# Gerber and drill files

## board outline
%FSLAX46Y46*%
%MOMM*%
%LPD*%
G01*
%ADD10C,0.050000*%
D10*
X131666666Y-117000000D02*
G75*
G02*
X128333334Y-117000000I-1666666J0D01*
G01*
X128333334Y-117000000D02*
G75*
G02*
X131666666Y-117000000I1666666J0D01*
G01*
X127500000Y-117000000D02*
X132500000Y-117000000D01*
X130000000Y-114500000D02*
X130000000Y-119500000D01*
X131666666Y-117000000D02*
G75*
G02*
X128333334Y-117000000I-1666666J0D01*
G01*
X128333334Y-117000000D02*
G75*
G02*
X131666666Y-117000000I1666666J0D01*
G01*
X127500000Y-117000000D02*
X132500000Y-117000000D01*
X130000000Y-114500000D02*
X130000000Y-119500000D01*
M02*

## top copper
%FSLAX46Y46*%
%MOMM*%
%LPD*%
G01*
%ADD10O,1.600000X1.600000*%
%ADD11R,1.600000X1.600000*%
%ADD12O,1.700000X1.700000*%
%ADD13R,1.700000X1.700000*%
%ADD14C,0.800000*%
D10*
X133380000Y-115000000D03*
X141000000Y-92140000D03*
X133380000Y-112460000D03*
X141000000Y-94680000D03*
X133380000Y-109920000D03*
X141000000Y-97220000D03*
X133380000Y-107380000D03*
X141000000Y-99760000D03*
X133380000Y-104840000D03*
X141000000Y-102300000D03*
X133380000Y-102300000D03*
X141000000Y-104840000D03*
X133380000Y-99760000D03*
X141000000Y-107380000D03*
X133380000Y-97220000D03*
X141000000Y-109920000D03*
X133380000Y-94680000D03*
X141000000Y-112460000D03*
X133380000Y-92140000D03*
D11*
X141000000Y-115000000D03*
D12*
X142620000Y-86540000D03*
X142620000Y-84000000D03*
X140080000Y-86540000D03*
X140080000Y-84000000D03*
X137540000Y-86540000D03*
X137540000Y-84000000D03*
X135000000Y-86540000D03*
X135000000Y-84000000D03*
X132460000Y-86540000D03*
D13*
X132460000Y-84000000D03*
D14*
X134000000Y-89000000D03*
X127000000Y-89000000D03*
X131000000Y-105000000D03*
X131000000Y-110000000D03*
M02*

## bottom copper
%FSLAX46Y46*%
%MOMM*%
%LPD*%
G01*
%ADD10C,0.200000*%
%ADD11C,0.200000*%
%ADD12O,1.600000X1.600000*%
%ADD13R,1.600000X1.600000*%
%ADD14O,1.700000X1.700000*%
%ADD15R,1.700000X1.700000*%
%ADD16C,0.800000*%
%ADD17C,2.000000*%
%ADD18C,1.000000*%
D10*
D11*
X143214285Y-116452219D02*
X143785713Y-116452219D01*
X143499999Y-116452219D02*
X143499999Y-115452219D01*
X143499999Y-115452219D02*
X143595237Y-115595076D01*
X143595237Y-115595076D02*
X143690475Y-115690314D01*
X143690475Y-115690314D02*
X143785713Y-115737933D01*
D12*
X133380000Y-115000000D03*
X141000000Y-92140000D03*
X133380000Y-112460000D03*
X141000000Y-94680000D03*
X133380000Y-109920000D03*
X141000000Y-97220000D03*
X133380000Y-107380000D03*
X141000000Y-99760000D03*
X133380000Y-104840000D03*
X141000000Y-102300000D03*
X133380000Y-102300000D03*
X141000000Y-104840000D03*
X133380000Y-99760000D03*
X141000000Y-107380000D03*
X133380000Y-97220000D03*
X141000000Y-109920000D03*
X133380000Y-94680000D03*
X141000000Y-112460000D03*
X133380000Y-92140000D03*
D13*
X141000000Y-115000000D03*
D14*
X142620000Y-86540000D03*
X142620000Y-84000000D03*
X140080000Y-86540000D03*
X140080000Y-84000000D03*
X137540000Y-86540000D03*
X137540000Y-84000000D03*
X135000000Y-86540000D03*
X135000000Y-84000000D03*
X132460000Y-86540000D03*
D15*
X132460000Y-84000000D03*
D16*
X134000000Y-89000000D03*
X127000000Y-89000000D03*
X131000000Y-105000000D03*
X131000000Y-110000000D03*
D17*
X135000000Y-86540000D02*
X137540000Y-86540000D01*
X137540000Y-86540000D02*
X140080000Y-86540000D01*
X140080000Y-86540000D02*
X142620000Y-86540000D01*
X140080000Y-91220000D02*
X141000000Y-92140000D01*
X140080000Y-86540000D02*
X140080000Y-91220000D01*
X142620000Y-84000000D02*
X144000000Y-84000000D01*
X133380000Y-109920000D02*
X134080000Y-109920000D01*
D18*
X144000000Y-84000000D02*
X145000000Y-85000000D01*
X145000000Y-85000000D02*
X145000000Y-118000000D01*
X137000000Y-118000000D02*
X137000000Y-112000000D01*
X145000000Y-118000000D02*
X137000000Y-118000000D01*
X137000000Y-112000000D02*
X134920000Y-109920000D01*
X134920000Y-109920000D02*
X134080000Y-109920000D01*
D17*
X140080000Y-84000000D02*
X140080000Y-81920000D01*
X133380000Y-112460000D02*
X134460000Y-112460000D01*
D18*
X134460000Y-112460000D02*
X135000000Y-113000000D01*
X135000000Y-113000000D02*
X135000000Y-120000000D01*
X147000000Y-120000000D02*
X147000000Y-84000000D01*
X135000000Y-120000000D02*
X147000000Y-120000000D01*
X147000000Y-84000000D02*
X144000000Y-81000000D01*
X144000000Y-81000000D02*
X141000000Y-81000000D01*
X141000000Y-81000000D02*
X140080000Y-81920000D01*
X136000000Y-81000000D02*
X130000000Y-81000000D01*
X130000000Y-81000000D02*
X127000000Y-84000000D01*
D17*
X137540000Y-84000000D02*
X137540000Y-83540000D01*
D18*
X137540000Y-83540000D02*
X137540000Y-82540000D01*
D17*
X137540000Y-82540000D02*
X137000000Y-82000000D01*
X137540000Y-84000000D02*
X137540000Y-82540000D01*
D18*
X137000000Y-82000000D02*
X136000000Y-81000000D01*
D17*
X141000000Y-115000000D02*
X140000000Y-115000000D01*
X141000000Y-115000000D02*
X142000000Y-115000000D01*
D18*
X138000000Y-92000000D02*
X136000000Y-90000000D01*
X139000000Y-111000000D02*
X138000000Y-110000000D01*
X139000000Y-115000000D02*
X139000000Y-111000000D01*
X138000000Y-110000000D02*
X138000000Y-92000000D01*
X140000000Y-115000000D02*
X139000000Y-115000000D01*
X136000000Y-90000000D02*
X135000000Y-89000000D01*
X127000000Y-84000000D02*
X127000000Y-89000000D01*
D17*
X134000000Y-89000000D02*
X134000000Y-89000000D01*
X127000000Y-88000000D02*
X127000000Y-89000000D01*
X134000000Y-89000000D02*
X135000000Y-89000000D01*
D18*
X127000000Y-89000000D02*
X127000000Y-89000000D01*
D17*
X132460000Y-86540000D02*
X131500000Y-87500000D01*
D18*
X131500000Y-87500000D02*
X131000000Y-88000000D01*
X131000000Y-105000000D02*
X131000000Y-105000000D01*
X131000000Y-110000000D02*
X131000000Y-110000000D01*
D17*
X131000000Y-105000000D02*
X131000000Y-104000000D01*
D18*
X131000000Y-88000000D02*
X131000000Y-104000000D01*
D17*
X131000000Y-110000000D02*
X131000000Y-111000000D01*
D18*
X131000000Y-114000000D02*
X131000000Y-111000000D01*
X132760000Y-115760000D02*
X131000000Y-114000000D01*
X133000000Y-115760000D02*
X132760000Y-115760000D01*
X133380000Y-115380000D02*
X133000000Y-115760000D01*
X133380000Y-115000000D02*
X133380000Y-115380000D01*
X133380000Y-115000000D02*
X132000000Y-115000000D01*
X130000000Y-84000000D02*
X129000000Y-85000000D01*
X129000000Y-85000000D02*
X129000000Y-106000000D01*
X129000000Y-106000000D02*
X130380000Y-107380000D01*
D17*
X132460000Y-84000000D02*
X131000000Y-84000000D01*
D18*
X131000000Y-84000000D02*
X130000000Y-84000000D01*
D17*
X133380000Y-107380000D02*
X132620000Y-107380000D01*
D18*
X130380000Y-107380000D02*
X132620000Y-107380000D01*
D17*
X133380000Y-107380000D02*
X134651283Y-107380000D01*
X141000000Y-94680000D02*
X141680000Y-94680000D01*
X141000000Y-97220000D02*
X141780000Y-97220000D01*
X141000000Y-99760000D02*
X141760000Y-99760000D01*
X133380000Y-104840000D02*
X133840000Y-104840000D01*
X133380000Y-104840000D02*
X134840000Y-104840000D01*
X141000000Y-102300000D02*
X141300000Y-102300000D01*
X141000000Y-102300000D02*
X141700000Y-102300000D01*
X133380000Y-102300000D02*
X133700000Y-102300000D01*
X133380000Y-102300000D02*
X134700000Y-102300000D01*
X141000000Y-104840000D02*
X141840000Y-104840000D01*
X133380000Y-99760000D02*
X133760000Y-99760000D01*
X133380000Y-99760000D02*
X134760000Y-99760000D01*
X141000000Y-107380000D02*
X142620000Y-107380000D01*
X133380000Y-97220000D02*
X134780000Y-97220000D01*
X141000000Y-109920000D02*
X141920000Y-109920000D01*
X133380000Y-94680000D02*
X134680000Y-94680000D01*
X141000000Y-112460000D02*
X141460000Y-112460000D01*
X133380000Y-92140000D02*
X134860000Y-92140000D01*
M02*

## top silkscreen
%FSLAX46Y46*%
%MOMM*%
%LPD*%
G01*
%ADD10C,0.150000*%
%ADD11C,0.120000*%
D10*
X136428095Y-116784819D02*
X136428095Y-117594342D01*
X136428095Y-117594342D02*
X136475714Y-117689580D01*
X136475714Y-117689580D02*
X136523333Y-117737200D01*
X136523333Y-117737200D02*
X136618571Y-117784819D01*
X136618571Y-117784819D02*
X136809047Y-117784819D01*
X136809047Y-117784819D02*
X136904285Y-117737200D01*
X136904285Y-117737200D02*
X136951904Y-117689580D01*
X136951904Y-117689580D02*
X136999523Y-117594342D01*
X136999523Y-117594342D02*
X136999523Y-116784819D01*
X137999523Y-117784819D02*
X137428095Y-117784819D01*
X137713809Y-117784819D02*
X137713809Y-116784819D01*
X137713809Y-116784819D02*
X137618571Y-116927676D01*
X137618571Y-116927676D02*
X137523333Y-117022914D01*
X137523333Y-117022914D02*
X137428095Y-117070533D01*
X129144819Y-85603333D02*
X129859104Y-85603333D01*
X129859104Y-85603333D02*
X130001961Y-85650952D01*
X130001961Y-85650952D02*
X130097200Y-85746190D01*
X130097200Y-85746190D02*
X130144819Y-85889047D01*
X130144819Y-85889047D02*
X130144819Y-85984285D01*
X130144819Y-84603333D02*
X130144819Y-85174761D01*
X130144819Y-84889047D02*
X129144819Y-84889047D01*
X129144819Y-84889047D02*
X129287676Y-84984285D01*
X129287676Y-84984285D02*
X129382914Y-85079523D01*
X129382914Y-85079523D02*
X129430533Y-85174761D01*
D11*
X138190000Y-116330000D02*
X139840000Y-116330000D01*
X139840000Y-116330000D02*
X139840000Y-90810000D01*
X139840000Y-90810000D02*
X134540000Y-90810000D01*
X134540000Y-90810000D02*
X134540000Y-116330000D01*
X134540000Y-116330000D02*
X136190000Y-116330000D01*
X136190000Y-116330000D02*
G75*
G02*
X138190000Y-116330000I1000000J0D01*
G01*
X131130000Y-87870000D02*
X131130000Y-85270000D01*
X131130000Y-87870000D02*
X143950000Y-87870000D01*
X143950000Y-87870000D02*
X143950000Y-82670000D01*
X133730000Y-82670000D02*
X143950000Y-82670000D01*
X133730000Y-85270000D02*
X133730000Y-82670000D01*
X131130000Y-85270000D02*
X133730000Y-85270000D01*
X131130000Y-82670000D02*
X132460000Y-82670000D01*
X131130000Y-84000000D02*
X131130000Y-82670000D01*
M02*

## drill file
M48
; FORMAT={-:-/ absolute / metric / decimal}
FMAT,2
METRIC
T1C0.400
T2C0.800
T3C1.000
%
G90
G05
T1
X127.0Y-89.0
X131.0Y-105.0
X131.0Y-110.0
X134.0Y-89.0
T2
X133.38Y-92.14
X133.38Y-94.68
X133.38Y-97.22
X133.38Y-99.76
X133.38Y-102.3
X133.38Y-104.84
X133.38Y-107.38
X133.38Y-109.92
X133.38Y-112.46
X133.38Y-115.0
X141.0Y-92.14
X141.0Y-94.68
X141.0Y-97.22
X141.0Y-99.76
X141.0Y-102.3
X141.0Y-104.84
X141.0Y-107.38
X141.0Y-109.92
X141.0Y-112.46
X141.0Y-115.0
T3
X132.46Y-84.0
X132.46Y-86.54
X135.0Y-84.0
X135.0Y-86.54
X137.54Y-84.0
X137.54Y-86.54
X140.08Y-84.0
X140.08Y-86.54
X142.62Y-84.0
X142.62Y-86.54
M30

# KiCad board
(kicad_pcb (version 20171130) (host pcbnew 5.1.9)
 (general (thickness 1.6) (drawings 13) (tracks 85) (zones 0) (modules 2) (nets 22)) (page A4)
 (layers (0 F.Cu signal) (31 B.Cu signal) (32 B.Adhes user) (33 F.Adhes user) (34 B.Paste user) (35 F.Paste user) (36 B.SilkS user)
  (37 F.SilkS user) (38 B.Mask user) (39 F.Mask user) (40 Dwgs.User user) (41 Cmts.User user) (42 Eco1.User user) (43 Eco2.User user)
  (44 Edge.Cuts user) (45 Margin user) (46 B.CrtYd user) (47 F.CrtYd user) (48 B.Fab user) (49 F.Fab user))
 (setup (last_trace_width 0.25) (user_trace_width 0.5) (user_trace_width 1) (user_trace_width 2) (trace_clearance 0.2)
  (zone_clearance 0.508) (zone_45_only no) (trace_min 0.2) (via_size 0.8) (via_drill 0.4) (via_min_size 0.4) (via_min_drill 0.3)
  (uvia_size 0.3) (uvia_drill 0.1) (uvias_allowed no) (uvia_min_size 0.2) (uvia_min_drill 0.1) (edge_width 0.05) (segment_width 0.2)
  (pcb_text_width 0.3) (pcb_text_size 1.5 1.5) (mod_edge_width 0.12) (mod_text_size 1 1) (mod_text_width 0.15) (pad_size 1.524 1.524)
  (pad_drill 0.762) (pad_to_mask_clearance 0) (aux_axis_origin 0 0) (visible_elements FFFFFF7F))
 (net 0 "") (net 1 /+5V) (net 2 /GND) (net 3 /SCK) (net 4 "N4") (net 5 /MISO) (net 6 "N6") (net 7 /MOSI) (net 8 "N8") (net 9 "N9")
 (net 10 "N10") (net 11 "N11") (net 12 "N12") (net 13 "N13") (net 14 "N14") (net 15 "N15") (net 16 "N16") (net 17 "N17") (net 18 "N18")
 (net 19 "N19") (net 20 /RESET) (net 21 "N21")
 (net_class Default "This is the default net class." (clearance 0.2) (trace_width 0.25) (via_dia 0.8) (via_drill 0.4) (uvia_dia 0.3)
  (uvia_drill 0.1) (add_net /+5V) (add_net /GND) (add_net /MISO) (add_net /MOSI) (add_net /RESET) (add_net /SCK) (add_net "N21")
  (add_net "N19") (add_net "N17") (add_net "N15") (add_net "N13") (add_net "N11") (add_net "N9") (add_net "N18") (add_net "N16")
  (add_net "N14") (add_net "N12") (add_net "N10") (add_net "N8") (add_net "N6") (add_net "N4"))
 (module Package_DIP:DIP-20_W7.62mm (layer F.Cu) (at 141 115 180)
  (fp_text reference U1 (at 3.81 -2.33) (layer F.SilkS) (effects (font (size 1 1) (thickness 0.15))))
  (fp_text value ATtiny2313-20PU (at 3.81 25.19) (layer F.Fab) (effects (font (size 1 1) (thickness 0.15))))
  (fp_line (start 2.81 -1.33) (end 1.16 -1.33) (layer F.SilkS) (width 0.12))
  (fp_line (start 1.16 -1.33) (end 1.16 24.19) (layer F.SilkS) (width 0.12))
  (fp_line (start 1.16 24.19) (end 6.46 24.19) (layer F.SilkS) (width 0.12))
  (fp_line (start 6.46 24.19) (end 6.46 -1.33) (layer F.SilkS) (width 0.12))
  (fp_line (start 6.46 -1.33) (end 4.81 -1.33) (layer F.SilkS) (width 0.12))
  (fp_arc (start 3.81 -1.33) (end 2.81 -1.33) (angle -180) (layer F.SilkS) (width 0.12))
  (pad 20 thru_hole oval (at 7.62 0 180) (size 1.6 1.6) (drill 0.8) (layers *.Cu *.Mask) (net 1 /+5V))
  (pad 10 thru_hole oval (at 0 22.86 180) (size 1.6 1.6) (drill 0.8) (layers *.Cu *.Mask) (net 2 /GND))
  (pad 19 thru_hole oval (at 7.62 2.54 180) (size 1.6 1.6) (drill 0.8) (layers *.Cu *.Mask) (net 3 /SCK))
  (pad 9 thru_hole oval (at 0 20.32 180) (size 1.6 1.6) (drill 0.8) (layers *.Cu *.Mask) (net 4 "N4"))
  (pad 18 thru_hole oval (at 7.62 5.08 180) (size 1.6 1.6) (drill 0.8) (layers *.Cu *.Mask) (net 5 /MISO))
  (pad 8 thru_hole oval (at 0 17.78 180) (size 1.6 1.6) (drill 0.8) (layers *.Cu *.Mask) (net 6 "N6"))
  (pad 17 thru_hole oval (at 7.62 7.62 180) (size 1.6 1.6) (drill 0.8) (layers *.Cu *.Mask) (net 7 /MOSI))
  (pad 7 thru_hole oval (at 0 15.24 180) (size 1.6 1.6) (drill 0.8) (layers *.Cu *.Mask) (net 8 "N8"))
  (pad 16 thru_hole oval (at 7.62 10.16 180) (size 1.6 1.6) (drill 0.8) (layers *.Cu *.Mask) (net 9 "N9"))
  (pad 6 thru_hole oval (at 0 12.7 180) (size 1.6 1.6) (drill 0.8) (layers *.Cu *.Mask) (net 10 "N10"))
  (pad 15 thru_hole oval (at 7.62 12.7 180) (size 1.6 1.6) (drill 0.8) (layers *.Cu *.Mask) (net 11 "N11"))
  (pad 5 thru_hole oval (at 0 10.16 180) (size 1.6 1.6) (drill 0.8) (layers *.Cu *.Mask) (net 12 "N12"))
  (pad 14 thru_hole oval (at 7.62 15.24 180) (size 1.6 1.6) (drill 0.8) (layers *.Cu *.Mask) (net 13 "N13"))
  (pad 4 thru_hole oval (at 0 7.62 180) (size 1.6 1.6) (drill 0.8) (layers *.Cu *.Mask) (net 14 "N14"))
  (pad 13 thru_hole oval (at 7.62 17.78 180) (size 1.6 1.6) (drill 0.8) (layers *.Cu *.Mask) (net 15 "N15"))
  (pad 3 thru_hole oval (at 0 5.08 180) (size 1.6 1.6) (drill 0.8) (layers *.Cu *.Mask) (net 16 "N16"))
  (pad 12 thru_hole oval (at 7.62 20.32 180) (size 1.6 1.6) (drill 0.8) (layers *.Cu *.Mask) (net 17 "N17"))
  (pad 2 thru_hole oval (at 0 2.54 180) (size 1.6 1.6) (drill 0.8) (layers *.Cu *.Mask) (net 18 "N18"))
  (pad 11 thru_hole oval (at 7.62 22.86 180) (size 1.6 1.6) (drill 0.8) (layers *.Cu *.Mask) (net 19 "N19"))
  (pad 1 thru_hole rect (at 0 0 180) (size 1.6 1.6) (drill 0.8) (layers *.Cu *.Mask) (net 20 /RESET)))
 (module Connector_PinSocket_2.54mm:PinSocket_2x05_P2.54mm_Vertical (layer F.Cu) (at 132.46 84 90)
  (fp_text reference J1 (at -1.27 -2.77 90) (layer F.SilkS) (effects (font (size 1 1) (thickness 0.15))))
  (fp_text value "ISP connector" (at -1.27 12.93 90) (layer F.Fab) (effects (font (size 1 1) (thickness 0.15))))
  (fp_line (start -3.87 -1.33) (end -1.27 -1.33) (layer F.SilkS) (width 0.12))
  (fp_line (start -3.87 -1.33) (end -3.87 11.49) (layer F.SilkS) (width 0.12))
  (fp_line (start -3.87 11.49) (end 1.33 11.49) (layer F.SilkS) (width 0.12))
  (fp_line (start 1.33 1.27) (end 1.33 11.49) (layer F.SilkS) (width 0.12))
  (fp_line (start -1.27 1.27) (end 1.33 1.27) (layer F.SilkS) (width 0.12))
  (fp_line (start -1.27 -1.33) (end -1.27 1.27) (layer F.SilkS) (width 0.12))
  (fp_line (start 1.33 -1.33) (end 1.33 0) (layer F.SilkS) (width 0.12))
  (fp_line (start 0 -1.33) (end 1.33 -1.33) (layer F.SilkS) (width 0.12))
  (pad 10 thru_hole oval (at -2.54 10.16 90) (size 1.7 1.7) (drill 1) (layers *.Cu *.Mask) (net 2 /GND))
  (pad 9 thru_hole oval (at 0 10.16 90) (size 1.7 1.7) (drill 1) (layers *.Cu *.Mask) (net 5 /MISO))
  (pad 8 thru_hole oval (at -2.54 7.62 90) (size 1.7 1.7) (drill 1) (layers *.Cu *.Mask) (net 2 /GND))
  (pad 7 thru_hole oval (at 0 7.62 90) (size 1.7 1.7) (drill 1) (layers *.Cu *.Mask) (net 3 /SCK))
  (pad 6 thru_hole oval (at -2.54 5.08 90) (size 1.7 1.7) (drill 1) (layers *.Cu *.Mask) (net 2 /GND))
  (pad 5 thru_hole oval (at 0 5.08 90) (size 1.7 1.7) (drill 1) (layers *.Cu *.Mask) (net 20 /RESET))
  (pad 4 thru_hole oval (at -2.54 2.54 90) (size 1.7 1.7) (drill 1) (layers *.Cu *.Mask) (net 2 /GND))
  (pad 3 thru_hole oval (at 0 2.54 90) (size 1.7 1.7) (drill 1) (layers *.Cu *.Mask) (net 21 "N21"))
  (pad 2 thru_hole oval (at -2.54 0 90) (size 1.7 1.7) (drill 1) (layers *.Cu *.Mask) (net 1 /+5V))
  (pad 1 thru_hole rect (at 0 0 90) (size 1.7 1.7) (drill 1) (layers *.Cu *.Mask) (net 7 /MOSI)))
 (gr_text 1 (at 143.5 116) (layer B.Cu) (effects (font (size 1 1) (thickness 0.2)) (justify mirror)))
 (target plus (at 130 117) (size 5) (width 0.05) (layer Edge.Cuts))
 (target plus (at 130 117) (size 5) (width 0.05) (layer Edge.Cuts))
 (segment (start 135 86.54) (end 137.54 86.54) (width 2) (layer B.Cu) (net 2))
 (segment (start 137.54 86.54) (end 140.08 86.54) (width 2) (layer B.Cu) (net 2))
 (segment (start 140.08 86.54) (end 142.62 86.54) (width 2) (layer B.Cu) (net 2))
 (segment (start 140.08 91.22) (end 141 92.14) (width 2) (layer B.Cu) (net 2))
 (segment (start 140.08 86.54) (end 140.08 91.22) (width 2) (layer B.Cu) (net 2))
 (segment (start 142.62 84) (end 144 84) (width 2) (layer B.Cu) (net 5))
 (segment (start 133.38 109.92) (end 134.08 109.92) (width 2) (layer B.Cu) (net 5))
 (segment (start 144 84) (end 145 85) (width 1) (layer B.Cu) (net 5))
 (segment (start 145 85) (end 145 118) (width 1) (layer B.Cu) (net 5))
 (segment (start 137 118) (end 137 112) (width 1) (layer B.Cu) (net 5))
 (segment (start 145 118) (end 137 118) (width 1) (layer B.Cu) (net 5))
 (segment (start 137 112) (end 134.92 109.92) (width 1) (layer B.Cu) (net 5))
 (segment (start 134.92 109.92) (end 134.08 109.92) (width 1) (layer B.Cu) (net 5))
 (segment (start 140.08 84) (end 140.08 81.92) (width 2) (layer B.Cu) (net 3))
 (segment (start 133.38 112.46) (end 134.46 112.46) (width 2) (layer B.Cu) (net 3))
 (segment (start 134.46 112.46) (end 135 113) (width 1) (layer B.Cu) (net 3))
 (segment (start 135 113) (end 135 120) (width 1) (layer B.Cu) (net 3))
 (segment (start 147 120) (end 147 84) (width 1) (layer B.Cu) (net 3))
 (segment (start 135 120) (end 147 120) (width 1) (layer B.Cu) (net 3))
 (segment (start 147 84) (end 144 81) (width 1) (layer B.Cu) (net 3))
 (segment (start 144 81) (end 141 81) (width 1) (layer B.Cu) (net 3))
 (segment (start 141 81) (end 140.08 81.92) (width 1) (layer B.Cu) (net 3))
 (segment (start 136 81) (end 130 81) (width 1) (layer B.Cu) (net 20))
 (segment (start 130 81) (end 127 84) (width 1) (layer B.Cu) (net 20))
 (segment (start 137.54 84) (end 137.54 83.54) (width 2) (layer B.Cu) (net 20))
 (segment (start 137.54 83.54) (end 137.54 82.54) (width 1) (layer B.Cu) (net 20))
 (segment (start 137.54 82.54) (end 137 82) (width 2) (layer B.Cu) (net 20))
 (segment (start 137.54 84) (end 137.54 82.54) (width 2) (layer B.Cu) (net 20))
 (segment (start 137 82) (end 136 81) (width 1) (layer B.Cu) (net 20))
 (segment (start 141 115) (end 140 115) (width 2) (layer B.Cu) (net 20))
 (segment (start 141 115) (end 142 115) (width 2) (layer B.Cu) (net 20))
 (segment (start 138 92) (end 136 90) (width 1) (layer B.Cu) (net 20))
 (segment (start 139 111) (end 138 110) (width 1) (layer B.Cu) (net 20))
 (segment (start 139 115) (end 139 111) (width 1) (layer B.Cu) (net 20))
 (segment (start 138 110) (end 138 92) (width 1) (layer B.Cu) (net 20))
 (segment (start 140 115) (end 139 115) (width 1) (layer B.Cu) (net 20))
 (segment (start 136 90) (end 135 89) (width 1) (layer B.Cu) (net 20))
 (segment (start 127 84) (end 127 89) (width 1) (layer B.Cu) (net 20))
 (segment (start 134 89) (end 134 89) (width 2) (layer B.Cu) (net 20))
 (segment (start 127 88) (end 127 89) (width 2) (layer B.Cu) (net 20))
 (segment (start 134 89) (end 135 89) (width 2) (layer B.Cu) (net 20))
 (via (at 134 89) (size 0.8) (drill 0.4) (layers F.Cu B.Cu) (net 20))
 (segment (start 127 89) (end 127 89) (width 1) (layer B.Cu) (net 20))
 (via (at 127 89) (size 0.8) (drill 0.4) (layers F.Cu B.Cu) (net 20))
 (segment (start 132.46 86.54) (end 131.5 87.5) (width 2) (layer B.Cu) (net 1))
 (segment (start 131.5 87.5) (end 131 88) (width 1) (layer B.Cu) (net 1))
 (segment (start 131 105) (end 131 105) (width 1) (layer B.Cu) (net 1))
 (via (at 131 105) (size 0.8) (drill 0.4) (layers F.Cu B.Cu) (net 1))
 (segment (start 131 110) (end 131 110) (width 1) (layer B.Cu) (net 1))
 (via (at 131 110) (size 0.8) (drill 0.4) (layers F.Cu B.Cu) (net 1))
 (segment (start 131 105) (end 131 104) (width 2) (layer B.Cu) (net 1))
 (segment (start 131 88) (end 131 104) (width 1) (layer B.Cu) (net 1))
 (segment (start 131 110) (end 131 111) (width 2) (layer B.Cu) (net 1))
 (segment (start 131 114) (end 131 111) (width 1) (layer B.Cu) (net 1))
 (segment (start 132.76 115.76) (end 131 114) (width 1) (layer B.Cu) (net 1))
 (segment (start 133 115.76) (end 132.76 115.76) (width 1) (layer B.Cu) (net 1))
 (segment (start 133.38 115.38) (end 133 115.76) (width 1) (layer B.Cu) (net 1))
 (segment (start 133.38 115) (end 133.38 115.38) (width 1) (layer B.Cu) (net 1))
 (segment (start 133.38 115) (end 132 115) (width 1) (layer B.Cu) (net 1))
 (segment (start 130 84) (end 129 85) (width 1) (layer B.Cu) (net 7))
 (segment (start 129 85) (end 129 106) (width 1) (layer B.Cu) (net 7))
 (segment (start 129 106) (end 130.38 107.38) (width 1) (layer B.Cu) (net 7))
 (segment (start 132.46 84) (end 131 84) (width 2) (layer B.Cu) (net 7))
 (segment (start 131 84) (end 130 84) (width 1) (layer B.Cu) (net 7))
 (segment (start 133.38 107.38) (end 132.62 107.38) (width 2) (layer B.Cu) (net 7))
 (segment (start 130.38 107.38) (end 132.62 107.38) (width 1) (layer B.Cu) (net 7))
 (segment (start 133.38 107.38) (end 134.651283 107.38) (width 2) (layer B.Cu) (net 7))
 (segment (start 141 94.68) (end 141.68 94.68) (width 2) (layer B.Cu) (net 4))
 (segment (start 141 97.22) (end 141.78 97.22) (width 2) (layer B.Cu) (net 6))
 (segment (start 141 99.76) (end 141.76 99.76) (width 2) (layer B.Cu) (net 8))
 (segment (start 133.38 104.84) (end 133.84 104.84) (width 2) (layer B.Cu) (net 9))
 (segment (start 133.38 104.84) (end 134.84 104.84) (width 2) (layer B.Cu) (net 9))
 (segment (start 141 102.3) (end 141.3 102.3) (width 2) (layer B.Cu) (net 10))
 (segment (start 141 102.3) (end 141.7 102.3) (width 2) (layer B.Cu) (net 10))
 (segment (start 133.38 102.3) (end 133.7 102.3) (width 2) (layer B.Cu) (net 11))
 (segment (start 133.38 102.3) (end 134.7 102.3) (width 2) (layer B.Cu) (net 11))
 (segment (start 141 104.84) (end 141.84 104.84) (width 2) (layer B.Cu) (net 12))
 (segment (start 133.38 99.76) (end 133.76 99.76) (width 2) (layer B.Cu) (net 13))
 (segment (start 133.38 99.76) (end 134.76 99.76) (width 2) (layer B.Cu) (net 13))
 (segment (start 141 107.38) (end 142.62 107.38) (width 2) (layer B.Cu) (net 14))
 (segment (start 133.38 97.22) (end 134.78 97.22) (width 2) (layer B.Cu) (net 15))
 (segment (start 141 109.92) (end 141.92 109.92) (width 2) (layer B.Cu) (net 16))
 (segment (start 133.38 94.68) (end 134.68 94.68) (width 2) (layer B.Cu) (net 17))
 (segment (start 141 112.46) (end 141.46 112.46) (width 2) (layer B.Cu) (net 18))
 (segment (start 133.38 92.14) (end 134.86 92.14) (width 2) (layer B.Cu) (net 19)))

